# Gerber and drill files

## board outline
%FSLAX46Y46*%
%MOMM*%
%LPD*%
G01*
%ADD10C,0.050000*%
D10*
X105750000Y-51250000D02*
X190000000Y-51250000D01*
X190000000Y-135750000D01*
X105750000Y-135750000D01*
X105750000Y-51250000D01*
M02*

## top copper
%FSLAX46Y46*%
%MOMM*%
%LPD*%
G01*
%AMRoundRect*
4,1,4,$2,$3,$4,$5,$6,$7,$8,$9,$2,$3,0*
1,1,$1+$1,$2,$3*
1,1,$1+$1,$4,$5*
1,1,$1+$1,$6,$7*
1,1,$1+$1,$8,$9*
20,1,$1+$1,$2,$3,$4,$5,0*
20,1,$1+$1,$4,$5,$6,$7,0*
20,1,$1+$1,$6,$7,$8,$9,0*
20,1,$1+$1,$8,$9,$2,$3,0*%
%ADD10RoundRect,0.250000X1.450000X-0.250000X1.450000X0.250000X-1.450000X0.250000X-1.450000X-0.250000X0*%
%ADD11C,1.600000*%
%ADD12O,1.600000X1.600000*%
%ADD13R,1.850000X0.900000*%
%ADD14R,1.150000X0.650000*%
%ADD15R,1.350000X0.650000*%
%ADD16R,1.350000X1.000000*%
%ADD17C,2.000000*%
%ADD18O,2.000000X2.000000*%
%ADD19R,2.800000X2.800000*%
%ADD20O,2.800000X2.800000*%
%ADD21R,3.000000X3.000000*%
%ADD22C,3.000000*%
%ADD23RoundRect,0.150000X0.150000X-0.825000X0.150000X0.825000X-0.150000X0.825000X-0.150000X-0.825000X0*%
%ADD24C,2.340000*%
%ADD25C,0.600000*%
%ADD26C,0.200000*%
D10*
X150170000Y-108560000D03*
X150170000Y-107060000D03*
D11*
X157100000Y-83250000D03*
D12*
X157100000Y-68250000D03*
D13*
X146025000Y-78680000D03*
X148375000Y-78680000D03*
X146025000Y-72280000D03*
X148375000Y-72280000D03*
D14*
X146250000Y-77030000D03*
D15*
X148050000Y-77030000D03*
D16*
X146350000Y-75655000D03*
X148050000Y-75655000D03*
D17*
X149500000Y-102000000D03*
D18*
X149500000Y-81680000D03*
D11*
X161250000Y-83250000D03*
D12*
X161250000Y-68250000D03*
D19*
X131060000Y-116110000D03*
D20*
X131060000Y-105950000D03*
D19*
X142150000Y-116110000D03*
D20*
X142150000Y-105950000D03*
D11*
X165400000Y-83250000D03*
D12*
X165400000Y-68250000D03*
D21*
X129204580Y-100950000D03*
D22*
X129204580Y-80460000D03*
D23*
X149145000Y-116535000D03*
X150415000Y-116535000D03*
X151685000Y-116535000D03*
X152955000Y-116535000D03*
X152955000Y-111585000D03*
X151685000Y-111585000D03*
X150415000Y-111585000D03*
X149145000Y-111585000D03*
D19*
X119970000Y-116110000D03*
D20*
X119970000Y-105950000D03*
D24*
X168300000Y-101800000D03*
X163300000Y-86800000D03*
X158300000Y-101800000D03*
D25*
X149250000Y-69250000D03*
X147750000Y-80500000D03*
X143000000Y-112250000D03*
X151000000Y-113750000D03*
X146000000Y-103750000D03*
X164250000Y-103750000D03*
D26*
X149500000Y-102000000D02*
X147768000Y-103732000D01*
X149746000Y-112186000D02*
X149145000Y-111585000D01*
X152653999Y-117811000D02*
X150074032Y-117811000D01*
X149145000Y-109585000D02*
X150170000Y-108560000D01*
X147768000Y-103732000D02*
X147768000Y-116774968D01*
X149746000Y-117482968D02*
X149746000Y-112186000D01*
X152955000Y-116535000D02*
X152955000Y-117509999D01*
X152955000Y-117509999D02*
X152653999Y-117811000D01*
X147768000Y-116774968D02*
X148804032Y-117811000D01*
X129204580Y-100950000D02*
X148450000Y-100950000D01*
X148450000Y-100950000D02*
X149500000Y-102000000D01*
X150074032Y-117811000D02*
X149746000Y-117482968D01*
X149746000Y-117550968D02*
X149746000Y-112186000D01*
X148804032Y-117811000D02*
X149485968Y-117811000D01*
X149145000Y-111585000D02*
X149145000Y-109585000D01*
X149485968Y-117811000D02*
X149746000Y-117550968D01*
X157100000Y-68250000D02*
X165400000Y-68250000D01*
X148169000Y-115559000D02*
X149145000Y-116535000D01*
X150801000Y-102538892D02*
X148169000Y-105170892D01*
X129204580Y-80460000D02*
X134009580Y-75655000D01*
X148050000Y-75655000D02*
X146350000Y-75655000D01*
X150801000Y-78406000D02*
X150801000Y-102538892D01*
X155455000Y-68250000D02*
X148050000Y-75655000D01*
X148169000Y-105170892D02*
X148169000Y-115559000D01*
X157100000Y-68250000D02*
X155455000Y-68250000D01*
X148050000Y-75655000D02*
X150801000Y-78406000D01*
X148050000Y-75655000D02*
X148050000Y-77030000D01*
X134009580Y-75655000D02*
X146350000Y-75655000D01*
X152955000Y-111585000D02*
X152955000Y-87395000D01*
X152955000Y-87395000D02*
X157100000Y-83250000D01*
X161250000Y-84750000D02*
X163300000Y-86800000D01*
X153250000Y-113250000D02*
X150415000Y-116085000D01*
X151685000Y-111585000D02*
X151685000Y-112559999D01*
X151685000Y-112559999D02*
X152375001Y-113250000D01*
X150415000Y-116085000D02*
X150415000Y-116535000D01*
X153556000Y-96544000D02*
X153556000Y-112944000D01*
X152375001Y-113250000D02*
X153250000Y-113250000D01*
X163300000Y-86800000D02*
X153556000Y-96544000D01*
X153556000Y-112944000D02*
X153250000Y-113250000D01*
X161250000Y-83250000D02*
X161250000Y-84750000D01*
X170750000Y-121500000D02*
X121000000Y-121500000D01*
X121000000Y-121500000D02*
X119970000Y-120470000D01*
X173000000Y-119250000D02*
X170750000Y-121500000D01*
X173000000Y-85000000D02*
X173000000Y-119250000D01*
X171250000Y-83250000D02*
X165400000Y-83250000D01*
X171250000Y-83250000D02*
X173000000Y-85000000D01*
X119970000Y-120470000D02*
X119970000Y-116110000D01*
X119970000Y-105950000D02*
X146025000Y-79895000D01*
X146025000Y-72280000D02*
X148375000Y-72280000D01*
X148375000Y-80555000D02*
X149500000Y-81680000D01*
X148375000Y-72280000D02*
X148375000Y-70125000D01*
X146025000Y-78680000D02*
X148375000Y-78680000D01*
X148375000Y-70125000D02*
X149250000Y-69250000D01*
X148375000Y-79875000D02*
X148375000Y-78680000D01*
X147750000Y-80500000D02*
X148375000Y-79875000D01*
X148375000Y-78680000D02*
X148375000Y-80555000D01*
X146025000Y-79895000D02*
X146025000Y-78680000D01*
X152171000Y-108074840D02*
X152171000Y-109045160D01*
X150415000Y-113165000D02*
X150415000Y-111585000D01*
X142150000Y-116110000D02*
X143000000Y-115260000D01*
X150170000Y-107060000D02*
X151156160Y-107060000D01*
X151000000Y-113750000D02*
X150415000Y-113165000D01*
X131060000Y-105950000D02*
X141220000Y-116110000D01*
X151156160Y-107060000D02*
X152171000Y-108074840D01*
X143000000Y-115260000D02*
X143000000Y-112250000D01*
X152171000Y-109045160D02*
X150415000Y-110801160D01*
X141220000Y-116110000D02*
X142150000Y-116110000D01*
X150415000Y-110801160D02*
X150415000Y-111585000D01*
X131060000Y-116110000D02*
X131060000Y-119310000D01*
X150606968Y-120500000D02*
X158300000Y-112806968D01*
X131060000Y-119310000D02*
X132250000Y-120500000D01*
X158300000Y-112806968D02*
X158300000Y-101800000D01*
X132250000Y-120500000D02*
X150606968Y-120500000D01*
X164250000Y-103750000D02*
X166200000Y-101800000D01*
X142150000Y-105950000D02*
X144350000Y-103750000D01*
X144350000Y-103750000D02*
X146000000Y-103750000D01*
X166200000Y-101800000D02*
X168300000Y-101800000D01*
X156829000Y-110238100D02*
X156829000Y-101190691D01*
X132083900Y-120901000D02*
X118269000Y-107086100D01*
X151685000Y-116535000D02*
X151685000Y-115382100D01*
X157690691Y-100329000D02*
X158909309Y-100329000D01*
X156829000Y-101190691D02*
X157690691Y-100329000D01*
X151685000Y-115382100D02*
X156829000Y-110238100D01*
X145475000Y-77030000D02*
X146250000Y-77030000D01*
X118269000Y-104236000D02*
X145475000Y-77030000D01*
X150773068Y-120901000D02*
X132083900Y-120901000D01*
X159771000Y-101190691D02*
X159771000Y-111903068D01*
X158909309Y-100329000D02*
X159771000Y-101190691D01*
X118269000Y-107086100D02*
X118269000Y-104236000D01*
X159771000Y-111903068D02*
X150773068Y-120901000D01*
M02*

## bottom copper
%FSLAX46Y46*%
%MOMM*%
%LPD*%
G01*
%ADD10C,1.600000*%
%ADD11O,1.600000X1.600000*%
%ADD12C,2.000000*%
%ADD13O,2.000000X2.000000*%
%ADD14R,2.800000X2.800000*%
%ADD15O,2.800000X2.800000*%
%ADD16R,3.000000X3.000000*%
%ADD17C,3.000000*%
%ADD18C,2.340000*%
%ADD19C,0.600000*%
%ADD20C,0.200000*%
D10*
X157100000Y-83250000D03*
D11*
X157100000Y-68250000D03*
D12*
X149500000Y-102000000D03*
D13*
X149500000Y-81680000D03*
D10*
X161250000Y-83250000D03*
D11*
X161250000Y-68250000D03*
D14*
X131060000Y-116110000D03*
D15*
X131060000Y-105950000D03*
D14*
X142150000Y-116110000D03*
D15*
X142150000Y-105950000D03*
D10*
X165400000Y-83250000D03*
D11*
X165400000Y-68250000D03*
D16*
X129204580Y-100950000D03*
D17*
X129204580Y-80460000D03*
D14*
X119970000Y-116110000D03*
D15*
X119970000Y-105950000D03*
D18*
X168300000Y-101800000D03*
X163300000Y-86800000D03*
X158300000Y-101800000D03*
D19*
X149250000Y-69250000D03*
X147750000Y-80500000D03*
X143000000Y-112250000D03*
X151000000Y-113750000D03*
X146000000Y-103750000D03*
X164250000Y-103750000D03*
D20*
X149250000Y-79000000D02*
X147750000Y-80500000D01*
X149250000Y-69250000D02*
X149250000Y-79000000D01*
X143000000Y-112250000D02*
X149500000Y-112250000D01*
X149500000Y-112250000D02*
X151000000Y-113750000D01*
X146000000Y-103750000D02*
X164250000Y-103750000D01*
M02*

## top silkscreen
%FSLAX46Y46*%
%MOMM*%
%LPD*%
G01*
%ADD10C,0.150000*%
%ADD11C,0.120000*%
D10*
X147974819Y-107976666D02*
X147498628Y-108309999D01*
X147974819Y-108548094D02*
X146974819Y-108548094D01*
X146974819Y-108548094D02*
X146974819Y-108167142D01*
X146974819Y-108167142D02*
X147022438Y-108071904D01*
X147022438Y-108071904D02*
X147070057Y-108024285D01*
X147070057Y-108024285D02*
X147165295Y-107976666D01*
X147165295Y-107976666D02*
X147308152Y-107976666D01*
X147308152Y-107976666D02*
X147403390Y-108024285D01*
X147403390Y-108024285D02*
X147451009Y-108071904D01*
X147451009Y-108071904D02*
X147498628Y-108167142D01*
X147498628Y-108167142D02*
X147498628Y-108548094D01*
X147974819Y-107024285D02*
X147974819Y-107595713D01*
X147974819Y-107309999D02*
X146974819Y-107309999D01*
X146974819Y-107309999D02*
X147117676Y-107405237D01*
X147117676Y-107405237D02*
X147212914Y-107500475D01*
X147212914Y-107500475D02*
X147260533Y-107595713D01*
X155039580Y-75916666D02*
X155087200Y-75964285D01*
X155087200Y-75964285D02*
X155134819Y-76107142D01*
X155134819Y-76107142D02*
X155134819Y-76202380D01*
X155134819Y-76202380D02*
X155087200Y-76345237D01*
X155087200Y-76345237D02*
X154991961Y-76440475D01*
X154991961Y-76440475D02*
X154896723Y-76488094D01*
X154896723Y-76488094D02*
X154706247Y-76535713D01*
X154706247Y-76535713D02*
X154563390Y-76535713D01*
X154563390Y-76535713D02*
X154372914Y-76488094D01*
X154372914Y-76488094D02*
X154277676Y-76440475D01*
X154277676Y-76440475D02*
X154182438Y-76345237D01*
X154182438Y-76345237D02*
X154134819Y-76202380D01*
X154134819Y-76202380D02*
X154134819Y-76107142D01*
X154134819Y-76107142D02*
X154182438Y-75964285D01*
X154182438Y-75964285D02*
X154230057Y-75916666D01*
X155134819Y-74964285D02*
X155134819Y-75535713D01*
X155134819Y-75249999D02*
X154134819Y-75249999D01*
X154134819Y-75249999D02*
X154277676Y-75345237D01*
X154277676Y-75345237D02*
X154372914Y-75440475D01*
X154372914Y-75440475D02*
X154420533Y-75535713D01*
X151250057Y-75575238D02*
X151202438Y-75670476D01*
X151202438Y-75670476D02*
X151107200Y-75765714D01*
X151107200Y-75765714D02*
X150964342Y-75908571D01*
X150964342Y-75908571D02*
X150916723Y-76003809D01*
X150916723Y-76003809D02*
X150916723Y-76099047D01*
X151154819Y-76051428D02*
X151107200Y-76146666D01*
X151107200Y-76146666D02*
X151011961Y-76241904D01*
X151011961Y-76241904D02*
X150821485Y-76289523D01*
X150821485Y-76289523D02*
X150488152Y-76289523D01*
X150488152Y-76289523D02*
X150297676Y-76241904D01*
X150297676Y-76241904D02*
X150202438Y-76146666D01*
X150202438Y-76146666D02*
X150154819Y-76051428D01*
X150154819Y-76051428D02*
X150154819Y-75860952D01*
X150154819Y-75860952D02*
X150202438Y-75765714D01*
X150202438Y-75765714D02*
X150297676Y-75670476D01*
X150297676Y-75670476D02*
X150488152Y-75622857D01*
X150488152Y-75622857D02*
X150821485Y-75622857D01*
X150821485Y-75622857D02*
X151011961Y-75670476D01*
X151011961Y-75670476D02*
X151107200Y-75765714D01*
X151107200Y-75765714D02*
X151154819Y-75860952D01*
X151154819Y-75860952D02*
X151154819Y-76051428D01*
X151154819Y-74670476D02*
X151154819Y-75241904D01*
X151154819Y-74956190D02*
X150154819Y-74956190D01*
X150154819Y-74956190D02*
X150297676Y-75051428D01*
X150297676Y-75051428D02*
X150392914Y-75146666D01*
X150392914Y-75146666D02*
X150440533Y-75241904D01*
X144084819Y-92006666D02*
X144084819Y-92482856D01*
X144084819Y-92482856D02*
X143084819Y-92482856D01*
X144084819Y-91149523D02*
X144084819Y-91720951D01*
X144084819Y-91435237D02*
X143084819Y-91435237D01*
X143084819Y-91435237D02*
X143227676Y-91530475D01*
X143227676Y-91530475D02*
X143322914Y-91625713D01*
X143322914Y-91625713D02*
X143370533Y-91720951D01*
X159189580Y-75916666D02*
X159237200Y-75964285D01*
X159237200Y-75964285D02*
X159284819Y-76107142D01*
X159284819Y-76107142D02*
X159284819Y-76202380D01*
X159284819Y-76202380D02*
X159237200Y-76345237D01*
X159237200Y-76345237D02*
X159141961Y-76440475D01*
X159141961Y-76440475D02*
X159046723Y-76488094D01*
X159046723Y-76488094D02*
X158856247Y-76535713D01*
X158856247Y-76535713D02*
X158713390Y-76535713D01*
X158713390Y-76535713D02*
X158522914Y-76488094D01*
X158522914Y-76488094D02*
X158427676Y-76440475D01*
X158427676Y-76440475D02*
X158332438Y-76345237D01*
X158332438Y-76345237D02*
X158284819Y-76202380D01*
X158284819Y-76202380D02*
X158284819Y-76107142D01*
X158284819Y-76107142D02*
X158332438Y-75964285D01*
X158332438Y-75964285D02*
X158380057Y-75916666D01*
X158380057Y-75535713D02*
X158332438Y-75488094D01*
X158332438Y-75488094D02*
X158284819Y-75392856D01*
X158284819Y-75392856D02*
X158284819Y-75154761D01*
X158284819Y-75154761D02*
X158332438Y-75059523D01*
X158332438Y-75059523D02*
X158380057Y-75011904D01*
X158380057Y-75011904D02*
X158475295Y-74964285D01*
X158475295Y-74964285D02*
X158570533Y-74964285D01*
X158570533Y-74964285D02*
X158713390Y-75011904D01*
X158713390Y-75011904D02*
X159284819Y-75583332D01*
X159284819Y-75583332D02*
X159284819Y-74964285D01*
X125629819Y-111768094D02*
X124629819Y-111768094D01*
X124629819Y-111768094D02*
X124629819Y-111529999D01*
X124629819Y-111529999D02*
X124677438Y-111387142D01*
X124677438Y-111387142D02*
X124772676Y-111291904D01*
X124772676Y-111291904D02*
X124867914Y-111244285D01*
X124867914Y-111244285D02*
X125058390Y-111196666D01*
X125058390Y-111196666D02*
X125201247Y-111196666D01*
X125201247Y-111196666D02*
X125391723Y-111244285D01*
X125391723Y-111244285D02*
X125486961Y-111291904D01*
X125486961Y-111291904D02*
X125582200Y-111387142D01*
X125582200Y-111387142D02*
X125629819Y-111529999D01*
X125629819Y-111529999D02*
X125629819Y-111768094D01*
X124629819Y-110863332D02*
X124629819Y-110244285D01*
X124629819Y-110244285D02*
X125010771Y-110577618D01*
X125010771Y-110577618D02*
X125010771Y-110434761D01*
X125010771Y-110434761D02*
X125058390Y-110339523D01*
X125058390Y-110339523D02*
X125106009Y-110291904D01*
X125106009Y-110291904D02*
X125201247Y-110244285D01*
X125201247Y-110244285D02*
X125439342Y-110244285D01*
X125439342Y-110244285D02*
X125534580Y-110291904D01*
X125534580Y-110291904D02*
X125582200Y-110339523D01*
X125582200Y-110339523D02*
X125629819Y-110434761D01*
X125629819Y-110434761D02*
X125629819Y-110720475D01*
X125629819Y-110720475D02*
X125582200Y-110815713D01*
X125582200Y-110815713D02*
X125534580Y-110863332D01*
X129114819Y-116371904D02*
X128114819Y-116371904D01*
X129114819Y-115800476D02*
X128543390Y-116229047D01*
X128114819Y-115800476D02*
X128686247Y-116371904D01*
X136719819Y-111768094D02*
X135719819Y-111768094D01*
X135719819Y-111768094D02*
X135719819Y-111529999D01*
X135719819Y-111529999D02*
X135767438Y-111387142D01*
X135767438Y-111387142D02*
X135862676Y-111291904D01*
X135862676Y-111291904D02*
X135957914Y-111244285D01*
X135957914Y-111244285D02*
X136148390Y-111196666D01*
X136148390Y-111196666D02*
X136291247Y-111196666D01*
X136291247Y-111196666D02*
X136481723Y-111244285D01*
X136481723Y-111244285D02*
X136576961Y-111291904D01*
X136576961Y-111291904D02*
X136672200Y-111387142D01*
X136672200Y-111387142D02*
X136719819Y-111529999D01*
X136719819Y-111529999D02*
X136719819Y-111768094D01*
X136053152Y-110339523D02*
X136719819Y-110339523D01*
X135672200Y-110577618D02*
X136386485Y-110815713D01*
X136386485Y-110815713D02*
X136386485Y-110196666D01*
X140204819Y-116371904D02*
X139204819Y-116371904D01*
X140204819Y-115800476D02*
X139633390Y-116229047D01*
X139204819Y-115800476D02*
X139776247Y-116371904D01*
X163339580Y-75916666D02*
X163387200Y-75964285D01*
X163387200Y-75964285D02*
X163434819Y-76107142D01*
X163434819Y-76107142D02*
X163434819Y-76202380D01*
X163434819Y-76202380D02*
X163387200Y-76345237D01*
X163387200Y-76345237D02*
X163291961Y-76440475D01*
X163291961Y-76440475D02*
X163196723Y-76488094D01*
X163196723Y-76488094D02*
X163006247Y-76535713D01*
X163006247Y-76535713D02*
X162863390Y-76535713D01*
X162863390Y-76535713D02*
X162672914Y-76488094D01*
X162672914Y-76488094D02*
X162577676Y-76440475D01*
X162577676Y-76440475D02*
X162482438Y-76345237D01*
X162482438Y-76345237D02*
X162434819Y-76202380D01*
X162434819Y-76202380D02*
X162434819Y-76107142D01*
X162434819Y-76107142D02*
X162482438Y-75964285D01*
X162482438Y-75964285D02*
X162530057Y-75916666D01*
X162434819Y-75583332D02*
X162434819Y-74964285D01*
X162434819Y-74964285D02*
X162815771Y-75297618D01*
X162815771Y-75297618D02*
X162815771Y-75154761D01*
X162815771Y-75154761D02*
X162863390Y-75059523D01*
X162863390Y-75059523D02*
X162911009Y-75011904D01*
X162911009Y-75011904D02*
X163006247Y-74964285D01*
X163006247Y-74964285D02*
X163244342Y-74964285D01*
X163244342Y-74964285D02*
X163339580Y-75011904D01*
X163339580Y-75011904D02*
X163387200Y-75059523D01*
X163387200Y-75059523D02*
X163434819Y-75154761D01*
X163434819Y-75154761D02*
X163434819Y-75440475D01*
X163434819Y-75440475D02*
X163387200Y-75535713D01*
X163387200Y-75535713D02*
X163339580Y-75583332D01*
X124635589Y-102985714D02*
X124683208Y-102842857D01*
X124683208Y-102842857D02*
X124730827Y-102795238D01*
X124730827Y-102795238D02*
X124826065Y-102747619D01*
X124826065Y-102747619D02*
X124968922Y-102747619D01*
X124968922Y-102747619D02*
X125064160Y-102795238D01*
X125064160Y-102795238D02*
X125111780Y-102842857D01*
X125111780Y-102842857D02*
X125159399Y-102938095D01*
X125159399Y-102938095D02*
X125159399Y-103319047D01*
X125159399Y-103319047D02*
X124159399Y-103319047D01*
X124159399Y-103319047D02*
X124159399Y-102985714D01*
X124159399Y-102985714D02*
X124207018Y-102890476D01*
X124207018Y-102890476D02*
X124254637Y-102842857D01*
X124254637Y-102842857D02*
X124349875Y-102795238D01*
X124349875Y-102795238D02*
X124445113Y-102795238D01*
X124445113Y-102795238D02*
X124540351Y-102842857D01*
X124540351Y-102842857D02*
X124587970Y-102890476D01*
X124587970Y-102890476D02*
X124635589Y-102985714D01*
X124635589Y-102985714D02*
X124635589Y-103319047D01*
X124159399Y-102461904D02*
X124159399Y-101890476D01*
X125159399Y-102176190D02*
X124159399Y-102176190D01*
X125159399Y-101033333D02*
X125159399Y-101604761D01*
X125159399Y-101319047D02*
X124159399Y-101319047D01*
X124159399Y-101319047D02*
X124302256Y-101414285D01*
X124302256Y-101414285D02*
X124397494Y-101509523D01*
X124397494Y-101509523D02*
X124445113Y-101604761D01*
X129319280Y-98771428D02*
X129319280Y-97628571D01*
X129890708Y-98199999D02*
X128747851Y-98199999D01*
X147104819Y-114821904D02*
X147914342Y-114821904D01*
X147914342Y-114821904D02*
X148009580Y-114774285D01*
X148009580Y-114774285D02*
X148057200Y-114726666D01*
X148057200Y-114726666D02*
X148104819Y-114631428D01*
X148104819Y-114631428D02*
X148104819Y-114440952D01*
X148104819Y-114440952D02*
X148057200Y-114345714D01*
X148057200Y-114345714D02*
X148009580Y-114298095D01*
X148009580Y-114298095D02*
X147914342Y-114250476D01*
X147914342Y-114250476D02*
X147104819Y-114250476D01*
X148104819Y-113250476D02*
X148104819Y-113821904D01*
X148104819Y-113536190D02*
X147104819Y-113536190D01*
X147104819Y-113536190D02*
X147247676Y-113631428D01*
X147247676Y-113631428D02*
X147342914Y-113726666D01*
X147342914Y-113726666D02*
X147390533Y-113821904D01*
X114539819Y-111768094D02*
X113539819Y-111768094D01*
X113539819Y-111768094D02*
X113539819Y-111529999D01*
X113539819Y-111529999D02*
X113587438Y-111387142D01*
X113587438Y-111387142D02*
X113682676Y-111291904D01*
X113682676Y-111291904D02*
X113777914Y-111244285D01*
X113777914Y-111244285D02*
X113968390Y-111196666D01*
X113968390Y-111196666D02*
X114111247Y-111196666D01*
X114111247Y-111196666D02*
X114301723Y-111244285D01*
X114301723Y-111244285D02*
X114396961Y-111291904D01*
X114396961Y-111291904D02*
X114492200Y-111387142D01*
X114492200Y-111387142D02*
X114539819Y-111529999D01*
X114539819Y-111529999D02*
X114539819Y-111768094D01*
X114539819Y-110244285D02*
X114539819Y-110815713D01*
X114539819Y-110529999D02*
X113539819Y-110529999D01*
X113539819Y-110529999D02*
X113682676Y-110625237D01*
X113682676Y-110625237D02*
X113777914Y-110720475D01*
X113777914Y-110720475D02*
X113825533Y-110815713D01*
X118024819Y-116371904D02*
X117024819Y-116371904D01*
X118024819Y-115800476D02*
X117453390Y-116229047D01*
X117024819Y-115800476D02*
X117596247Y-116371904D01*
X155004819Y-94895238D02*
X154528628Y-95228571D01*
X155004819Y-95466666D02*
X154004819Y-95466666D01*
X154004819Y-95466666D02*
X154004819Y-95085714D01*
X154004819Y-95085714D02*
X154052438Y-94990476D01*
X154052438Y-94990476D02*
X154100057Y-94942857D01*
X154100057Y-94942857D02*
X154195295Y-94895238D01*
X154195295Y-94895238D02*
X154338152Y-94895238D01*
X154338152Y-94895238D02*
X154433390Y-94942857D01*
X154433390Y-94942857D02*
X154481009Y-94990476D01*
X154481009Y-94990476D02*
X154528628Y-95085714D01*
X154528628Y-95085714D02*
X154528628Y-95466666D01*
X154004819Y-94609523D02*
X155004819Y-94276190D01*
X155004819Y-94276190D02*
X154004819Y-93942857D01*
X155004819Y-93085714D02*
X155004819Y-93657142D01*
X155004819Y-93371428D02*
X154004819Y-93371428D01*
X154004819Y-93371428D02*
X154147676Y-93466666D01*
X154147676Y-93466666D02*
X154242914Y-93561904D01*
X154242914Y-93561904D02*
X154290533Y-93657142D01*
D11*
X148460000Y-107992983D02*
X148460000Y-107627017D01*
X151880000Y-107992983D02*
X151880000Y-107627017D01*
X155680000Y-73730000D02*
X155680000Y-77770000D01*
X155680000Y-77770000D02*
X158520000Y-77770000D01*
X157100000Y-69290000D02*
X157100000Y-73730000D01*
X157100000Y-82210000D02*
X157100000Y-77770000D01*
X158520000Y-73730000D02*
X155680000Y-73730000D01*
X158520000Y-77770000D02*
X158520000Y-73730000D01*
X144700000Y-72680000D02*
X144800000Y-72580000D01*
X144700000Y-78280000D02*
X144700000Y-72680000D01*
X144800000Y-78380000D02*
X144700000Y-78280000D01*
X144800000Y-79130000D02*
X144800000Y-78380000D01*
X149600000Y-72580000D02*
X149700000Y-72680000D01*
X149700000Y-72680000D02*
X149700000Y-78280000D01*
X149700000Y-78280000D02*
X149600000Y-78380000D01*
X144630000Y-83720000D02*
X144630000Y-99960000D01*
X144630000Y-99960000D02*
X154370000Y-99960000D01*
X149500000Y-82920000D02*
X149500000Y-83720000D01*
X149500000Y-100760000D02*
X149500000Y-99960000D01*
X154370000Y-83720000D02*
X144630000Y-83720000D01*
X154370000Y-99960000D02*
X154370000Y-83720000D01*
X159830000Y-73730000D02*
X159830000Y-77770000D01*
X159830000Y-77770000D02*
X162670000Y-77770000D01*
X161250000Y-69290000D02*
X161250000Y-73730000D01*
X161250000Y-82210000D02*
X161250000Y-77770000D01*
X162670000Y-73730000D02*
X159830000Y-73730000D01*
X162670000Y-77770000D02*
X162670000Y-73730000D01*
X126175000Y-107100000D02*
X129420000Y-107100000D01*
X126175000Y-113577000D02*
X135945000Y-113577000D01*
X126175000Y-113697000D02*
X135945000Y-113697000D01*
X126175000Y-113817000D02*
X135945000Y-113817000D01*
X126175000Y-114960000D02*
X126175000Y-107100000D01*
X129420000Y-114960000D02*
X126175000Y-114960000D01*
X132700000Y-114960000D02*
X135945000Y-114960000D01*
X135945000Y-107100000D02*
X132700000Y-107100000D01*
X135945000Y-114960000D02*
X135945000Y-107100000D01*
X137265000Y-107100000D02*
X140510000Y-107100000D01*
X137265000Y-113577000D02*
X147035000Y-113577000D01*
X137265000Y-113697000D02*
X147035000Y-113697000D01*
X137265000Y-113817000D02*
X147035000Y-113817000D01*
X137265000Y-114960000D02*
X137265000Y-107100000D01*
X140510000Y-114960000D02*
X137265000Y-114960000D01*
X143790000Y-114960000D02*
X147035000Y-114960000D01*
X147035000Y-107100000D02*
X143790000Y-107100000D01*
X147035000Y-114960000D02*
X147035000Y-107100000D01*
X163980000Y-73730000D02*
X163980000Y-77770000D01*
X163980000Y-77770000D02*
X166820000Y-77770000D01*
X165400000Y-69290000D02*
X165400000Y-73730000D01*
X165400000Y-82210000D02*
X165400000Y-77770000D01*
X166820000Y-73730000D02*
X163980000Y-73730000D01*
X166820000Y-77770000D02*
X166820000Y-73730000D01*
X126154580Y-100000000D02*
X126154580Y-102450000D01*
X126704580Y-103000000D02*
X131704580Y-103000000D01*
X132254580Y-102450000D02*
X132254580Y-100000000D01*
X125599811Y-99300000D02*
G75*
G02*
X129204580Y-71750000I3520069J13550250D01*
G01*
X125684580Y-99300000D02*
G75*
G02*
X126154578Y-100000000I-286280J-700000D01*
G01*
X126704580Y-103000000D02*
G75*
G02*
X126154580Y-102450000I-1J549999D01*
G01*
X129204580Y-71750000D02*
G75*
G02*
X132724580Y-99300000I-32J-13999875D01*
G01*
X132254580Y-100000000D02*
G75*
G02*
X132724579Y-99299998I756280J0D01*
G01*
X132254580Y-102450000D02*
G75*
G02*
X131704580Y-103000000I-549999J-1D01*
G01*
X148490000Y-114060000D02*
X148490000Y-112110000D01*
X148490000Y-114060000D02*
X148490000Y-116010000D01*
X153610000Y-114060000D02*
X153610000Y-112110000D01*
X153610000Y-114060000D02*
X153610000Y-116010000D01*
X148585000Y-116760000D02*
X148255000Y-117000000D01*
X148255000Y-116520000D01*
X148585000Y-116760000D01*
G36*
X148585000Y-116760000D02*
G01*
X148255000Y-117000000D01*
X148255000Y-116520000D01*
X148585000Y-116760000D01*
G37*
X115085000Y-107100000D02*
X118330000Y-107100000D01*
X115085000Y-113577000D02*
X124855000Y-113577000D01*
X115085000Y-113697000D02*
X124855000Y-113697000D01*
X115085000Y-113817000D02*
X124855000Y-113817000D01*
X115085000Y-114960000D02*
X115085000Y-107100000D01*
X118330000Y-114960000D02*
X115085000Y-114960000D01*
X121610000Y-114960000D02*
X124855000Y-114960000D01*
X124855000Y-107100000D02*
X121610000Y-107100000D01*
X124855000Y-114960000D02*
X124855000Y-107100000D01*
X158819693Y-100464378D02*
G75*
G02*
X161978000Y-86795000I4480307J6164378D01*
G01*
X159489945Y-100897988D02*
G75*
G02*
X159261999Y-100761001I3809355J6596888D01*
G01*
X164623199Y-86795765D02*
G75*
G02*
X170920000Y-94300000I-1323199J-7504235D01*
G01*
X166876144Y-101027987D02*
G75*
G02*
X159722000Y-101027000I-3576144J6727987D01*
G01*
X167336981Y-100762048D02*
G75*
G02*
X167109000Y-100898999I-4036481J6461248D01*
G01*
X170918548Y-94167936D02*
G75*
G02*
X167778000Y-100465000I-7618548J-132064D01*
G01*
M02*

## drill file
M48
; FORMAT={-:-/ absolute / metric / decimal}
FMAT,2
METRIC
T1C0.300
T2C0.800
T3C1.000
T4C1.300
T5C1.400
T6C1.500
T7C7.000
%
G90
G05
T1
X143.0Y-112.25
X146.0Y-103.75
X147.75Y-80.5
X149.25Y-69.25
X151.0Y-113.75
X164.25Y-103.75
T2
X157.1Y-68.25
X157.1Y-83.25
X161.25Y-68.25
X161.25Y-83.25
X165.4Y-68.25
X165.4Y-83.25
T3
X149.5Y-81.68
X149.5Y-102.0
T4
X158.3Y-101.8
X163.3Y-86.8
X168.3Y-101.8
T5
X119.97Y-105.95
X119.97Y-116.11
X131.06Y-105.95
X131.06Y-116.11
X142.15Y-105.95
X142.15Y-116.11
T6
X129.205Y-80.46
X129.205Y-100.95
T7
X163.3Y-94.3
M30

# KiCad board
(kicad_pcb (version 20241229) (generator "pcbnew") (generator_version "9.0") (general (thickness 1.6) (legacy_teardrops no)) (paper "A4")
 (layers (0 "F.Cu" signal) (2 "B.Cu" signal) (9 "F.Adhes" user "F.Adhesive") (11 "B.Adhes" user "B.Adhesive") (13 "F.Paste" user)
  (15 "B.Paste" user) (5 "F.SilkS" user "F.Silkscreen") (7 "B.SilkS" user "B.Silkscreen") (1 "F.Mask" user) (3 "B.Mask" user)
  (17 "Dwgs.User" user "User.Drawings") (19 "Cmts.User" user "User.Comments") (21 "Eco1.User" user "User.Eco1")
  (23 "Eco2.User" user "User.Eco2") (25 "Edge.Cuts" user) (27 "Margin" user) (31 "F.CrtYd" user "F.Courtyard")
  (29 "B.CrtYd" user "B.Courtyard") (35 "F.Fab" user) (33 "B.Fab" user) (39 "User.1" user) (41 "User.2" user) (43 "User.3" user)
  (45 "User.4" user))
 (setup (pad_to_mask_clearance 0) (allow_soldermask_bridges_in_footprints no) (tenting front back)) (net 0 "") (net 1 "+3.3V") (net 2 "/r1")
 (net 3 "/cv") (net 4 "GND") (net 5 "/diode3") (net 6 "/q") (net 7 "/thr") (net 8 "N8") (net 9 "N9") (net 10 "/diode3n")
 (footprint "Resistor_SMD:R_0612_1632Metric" (layer "F.Cu") (at 150.17 107.81 90)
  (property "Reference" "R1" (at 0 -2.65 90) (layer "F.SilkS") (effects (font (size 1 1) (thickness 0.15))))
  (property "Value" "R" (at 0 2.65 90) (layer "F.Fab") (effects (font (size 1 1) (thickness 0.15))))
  (fp_line (start -0.182983 -1.71) (end 0.182983 -1.71) (stroke (width 0.12) (type solid)) (layer "F.SilkS"))
  (fp_line (start -0.182983 1.71) (end 0.182983 1.71) (stroke (width 0.12) (type solid)) (layer "F.SilkS"))
  (pad "1" smd roundrect (at -0.75 0 90) (size 1 3.4) (layers "F.Cu" "F.Mask" "F.Paste") (roundrect_rratio 0.25) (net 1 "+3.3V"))
  (pad "2" smd roundrect (at 0.75 0 90) (size 1 3.4) (layers "F.Cu" "F.Mask" "F.Paste") (roundrect_rratio 0.25) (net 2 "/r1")))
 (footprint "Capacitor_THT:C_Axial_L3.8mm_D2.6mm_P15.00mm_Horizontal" (layer "F.Cu") (at 157.1 83.25 90)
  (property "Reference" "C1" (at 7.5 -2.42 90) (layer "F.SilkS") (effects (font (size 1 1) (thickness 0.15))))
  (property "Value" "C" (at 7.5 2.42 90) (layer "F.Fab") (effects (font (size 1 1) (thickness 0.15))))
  (fp_line (start 9.52 -1.42) (end 5.48 -1.42) (stroke (width 0.12) (type solid)) (layer "F.SilkS"))
  (fp_line (start 5.48 -1.42) (end 5.48 1.42) (stroke (width 0.12) (type solid)) (layer "F.SilkS"))
  (fp_line (start 13.96 0) (end 9.52 0) (stroke (width 0.12) (type solid)) (layer "F.SilkS"))
  (fp_line (start 1.04 0) (end 5.48 0) (stroke (width 0.12) (type solid)) (layer "F.SilkS"))
  (fp_line (start 9.52 1.42) (end 9.52 -1.42) (stroke (width 0.12) (type solid)) (layer "F.SilkS"))
  (fp_line (start 5.48 1.42) (end 9.52 1.42) (stroke (width 0.12) (type solid)) (layer "F.SilkS"))
  (pad "1" thru_hole circle (at 0 0 90) (size 1.6 1.6) (drill 0.8) (layers "*.Cu" "*.Mask") (remove_unused_layers no) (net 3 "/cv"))
  (pad "2" thru_hole oval (at 15 0 90) (size 1.6 1.6) (drill 0.8) (layers "*.Cu" "*.Mask") (remove_unused_layers no) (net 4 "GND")))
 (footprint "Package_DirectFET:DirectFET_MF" (layer "F.Cu") (at 147.2 75.48 90)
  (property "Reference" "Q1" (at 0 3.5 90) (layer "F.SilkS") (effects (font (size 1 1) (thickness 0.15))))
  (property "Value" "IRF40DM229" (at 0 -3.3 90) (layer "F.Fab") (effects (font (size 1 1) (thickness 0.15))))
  (fp_line (start 2.8 -2.5) (end 2.9 -2.4) (stroke (width 0.12) (type solid)) (layer "F.SilkS"))
  (fp_line (start -2.8 -2.5) (end 2.8 -2.5) (stroke (width 0.12) (type solid)) (layer "F.SilkS"))
  (fp_line (start -2.9 -2.4) (end -2.8 -2.5) (stroke (width 0.12) (type solid)) (layer "F.SilkS"))
  (fp_line (start -3.65 -2.4) (end -2.9 -2.4) (stroke (width 0.12) (type solid)) (layer "F.SilkS"))
  (fp_line (start 2.9 2.4) (end 2.8 2.5) (stroke (width 0.12) (type solid)) (layer "F.SilkS"))
  (fp_line (start 2.8 2.5) (end -2.8 2.5) (stroke (width 0.12) (type solid)) (layer "F.SilkS"))
  (fp_line (start -2.8 2.5) (end -2.9 2.4) (stroke (width 0.12) (type solid)) (layer "F.SilkS"))
  (pad "1" smd rect (at -3.2 -1.175 90) (size 0.9 1.85) (layers "F.Cu" "F.Mask" "F.Paste") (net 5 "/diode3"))
  (pad "1" smd rect (at -3.2 1.175 90) (size 0.9 1.85) (layers "F.Cu" "F.Mask" "F.Paste") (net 5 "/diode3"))
  (pad "1" smd rect (at 3.2 -1.175 90) (size 0.9 1.85) (layers "F.Cu" "F.Mask" "F.Paste") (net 5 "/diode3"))
  (pad "1" smd rect (at 3.2 1.175 90) (size 0.9 1.85) (layers "F.Cu" "F.Mask" "F.Paste") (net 5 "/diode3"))
  (pad "2" smd rect (at -1.55 -0.95 90) (size 0.65 1.15) (layers "F.Cu" "F.Mask" "F.Paste") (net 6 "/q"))
  (pad "3" smd rect (at -1.55 0.85 90) (size 0.65 1.35) (layers "F.Cu" "F.Mask" "F.Paste") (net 4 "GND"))
  (pad "3" smd rect (at -0.175 -0.85 90) (size 1 1.35) (layers "F.Cu" "F.Mask" "F.Paste") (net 4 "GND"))
  (pad "3" smd rect (at -0.175 0.85 90) (size 1 1.35) (layers "F.Cu" "F.Mask" "F.Paste") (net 4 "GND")))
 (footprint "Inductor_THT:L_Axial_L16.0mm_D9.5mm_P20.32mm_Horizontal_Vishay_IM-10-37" (layer "F.Cu") (at 149.5 102 90)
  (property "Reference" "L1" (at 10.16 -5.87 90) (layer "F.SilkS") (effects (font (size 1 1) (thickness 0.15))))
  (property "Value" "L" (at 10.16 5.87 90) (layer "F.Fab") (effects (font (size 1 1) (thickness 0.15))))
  (fp_line (start 18.28 -4.87) (end 2.04 -4.87) (stroke (width 0.12) (type solid)) (layer "F.SilkS"))
  (fp_line (start 2.04 -4.87) (end 2.04 4.87) (stroke (width 0.12) (type solid)) (layer "F.SilkS"))
  (fp_line (start 19.08 0) (end 18.28 0) (stroke (width 0.12) (type solid)) (layer "F.SilkS"))
  (fp_line (start 1.24 0) (end 2.04 0) (stroke (width 0.12) (type solid)) (layer "F.SilkS"))
  (fp_line (start 18.28 4.87) (end 18.28 -4.87) (stroke (width 0.12) (type solid)) (layer "F.SilkS"))
  (fp_line (start 2.04 4.87) (end 18.28 4.87) (stroke (width 0.12) (type solid)) (layer "F.SilkS"))
  (pad "1" thru_hole circle (at 0 0 90) (size 2 2) (drill 1) (layers "*.Cu" "*.Mask") (remove_unused_layers no) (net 1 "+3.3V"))
  (pad "2" thru_hole oval (at 20.32 0 90) (size 2 2) (drill 1) (layers "*.Cu" "*.Mask") (remove_unused_layers no) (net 5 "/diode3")))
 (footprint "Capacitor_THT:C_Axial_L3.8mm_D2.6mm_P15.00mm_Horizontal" (layer "F.Cu") (at 161.25 83.25 90)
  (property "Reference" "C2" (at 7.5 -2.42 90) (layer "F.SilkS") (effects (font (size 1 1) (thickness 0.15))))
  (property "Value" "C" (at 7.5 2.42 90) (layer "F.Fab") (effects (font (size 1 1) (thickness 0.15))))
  (fp_line (start 9.52 -1.42) (end 5.48 -1.42) (stroke (width 0.12) (type solid)) (layer "F.SilkS"))
  (fp_line (start 5.48 -1.42) (end 5.48 1.42) (stroke (width 0.12) (type solid)) (layer "F.SilkS"))
  (fp_line (start 13.96 0) (end 9.52 0) (stroke (width 0.12) (type solid)) (layer "F.SilkS"))
  (fp_line (start 1.04 0) (end 5.48 0) (stroke (width 0.12) (type solid)) (layer "F.SilkS"))
  (fp_line (start 9.52 1.42) (end 9.52 -1.42) (stroke (width 0.12) (type solid)) (layer "F.SilkS"))
  (fp_line (start 5.48 1.42) (end 9.52 1.42) (stroke (width 0.12) (type solid)) (layer "F.SilkS"))
  (pad "1" thru_hole circle (at 0 0 90) (size 1.6 1.6) (drill 0.8) (layers "*.Cu" "*.Mask") (remove_unused_layers no) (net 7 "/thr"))
  (pad "2" thru_hole oval (at 15 0 90) (size 1.6 1.6) (drill 0.8) (layers "*.Cu" "*.Mask") (remove_unused_layers no) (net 4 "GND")))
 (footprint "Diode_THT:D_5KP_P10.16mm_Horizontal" (layer "F.Cu") (at 131.06 116.11 90)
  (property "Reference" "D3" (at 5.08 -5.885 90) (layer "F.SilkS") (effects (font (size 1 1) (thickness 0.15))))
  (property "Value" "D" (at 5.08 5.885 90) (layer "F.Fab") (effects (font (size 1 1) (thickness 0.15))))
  (fp_line (start 9.01 -4.885) (end 9.01 -1.64) (stroke (width 0.12) (type solid)) (layer "F.SilkS"))
  (fp_line (start 2.533 -4.885) (end 2.533 4.885) (stroke (width 0.12) (type solid)) (layer "F.SilkS"))
  (fp_line (start 2.413 -4.885) (end 2.413 4.885) (stroke (width 0.12) (type solid)) (layer "F.SilkS"))
  (fp_line (start 2.293 -4.885) (end 2.293 4.885) (stroke (width 0.12) (type solid)) (layer "F.SilkS"))
  (fp_line (start 1.15 -4.885) (end 9.01 -4.885) (stroke (width 0.12) (type solid)) (layer "F.SilkS"))
  (fp_line (start 1.15 -1.64) (end 1.15 -4.885) (stroke (width 0.12) (type solid)) (layer "F.SilkS"))
  (fp_line (start 1.15 1.64) (end 1.15 4.885) (stroke (width 0.12) (type solid)) (layer "F.SilkS"))
  (fp_line (start 9.01 4.885) (end 9.01 1.64) (stroke (width 0.12) (type solid)) (layer "F.SilkS"))
  (fp_line (start 1.15 4.885) (end 9.01 4.885) (stroke (width 0.12) (type solid)) (layer "F.SilkS"))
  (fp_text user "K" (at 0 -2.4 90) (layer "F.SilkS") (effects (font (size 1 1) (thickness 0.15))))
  (pad "1" thru_hole rect (at 0 0 90) (size 2.8 2.8) (drill 1.4) (layers "*.Cu" "*.Mask") (remove_unused_layers no) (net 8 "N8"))
  (pad "2" thru_hole oval (at 10.16 0 90) (size 2.8 2.8) (drill 1.4) (layers "*.Cu" "*.Mask") (remove_unused_layers no) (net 2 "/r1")))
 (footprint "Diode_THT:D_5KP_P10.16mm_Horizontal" (layer "F.Cu") (at 142.15 116.11 90)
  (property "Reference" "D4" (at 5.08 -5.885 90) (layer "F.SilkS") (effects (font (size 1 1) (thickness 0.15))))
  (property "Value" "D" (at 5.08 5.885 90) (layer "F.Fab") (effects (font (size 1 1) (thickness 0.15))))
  (fp_line (start 9.01 -4.885) (end 9.01 -1.64) (stroke (width 0.12) (type solid)) (layer "F.SilkS"))
  (fp_line (start 2.533 -4.885) (end 2.533 4.885) (stroke (width 0.12) (type solid)) (layer "F.SilkS"))
  (fp_line (start 2.413 -4.885) (end 2.413 4.885) (stroke (width 0.12) (type solid)) (layer "F.SilkS"))
  (fp_line (start 2.293 -4.885) (end 2.293 4.885) (stroke (width 0.12) (type solid)) (layer "F.SilkS"))
  (fp_line (start 1.15 -4.885) (end 9.01 -4.885) (stroke (width 0.12) (type solid)) (layer "F.SilkS"))
  (fp_line (start 1.15 -1.64) (end 1.15 -4.885) (stroke (width 0.12) (type solid)) (layer "F.SilkS"))
  (fp_line (start 1.15 1.64) (end 1.15 4.885) (stroke (width 0.12) (type solid)) (layer "F.SilkS"))
  (fp_line (start 9.01 4.885) (end 9.01 1.64) (stroke (width 0.12) (type solid)) (layer "F.SilkS"))
  (fp_line (start 1.15 4.885) (end 9.01 4.885) (stroke (width 0.12) (type solid)) (layer "F.SilkS"))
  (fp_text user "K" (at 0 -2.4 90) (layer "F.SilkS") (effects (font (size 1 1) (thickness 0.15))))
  (pad "1" thru_hole rect (at 0 0 90) (size 2.8 2.8) (drill 1.4) (layers "*.Cu" "*.Mask") (remove_unused_layers no) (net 2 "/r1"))
  (pad "2" thru_hole oval (at 10.16 0 90) (size 2.8 2.8) (drill 1.4) (layers "*.Cu" "*.Mask") (remove_unused_layers no) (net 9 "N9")))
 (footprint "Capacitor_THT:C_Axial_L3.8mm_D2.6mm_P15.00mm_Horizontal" (layer "F.Cu") (at 165.4 83.25 90)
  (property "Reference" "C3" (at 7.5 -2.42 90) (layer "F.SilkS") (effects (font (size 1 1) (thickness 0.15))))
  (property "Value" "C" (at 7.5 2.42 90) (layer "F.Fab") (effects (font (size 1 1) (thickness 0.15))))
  (fp_line (start 9.52 -1.42) (end 5.48 -1.42) (stroke (width 0.12) (type solid)) (layer "F.SilkS"))
  (fp_line (start 5.48 -1.42) (end 5.48 1.42) (stroke (width 0.12) (type solid)) (layer "F.SilkS"))
  (fp_line (start 13.96 0) (end 9.52 0) (stroke (width 0.12) (type solid)) (layer "F.SilkS"))
  (fp_line (start 1.04 0) (end 5.48 0) (stroke (width 0.12) (type solid)) (layer "F.SilkS"))
  (fp_line (start 9.52 1.42) (end 9.52 -1.42) (stroke (width 0.12) (type solid)) (layer "F.SilkS"))
  (fp_line (start 5.48 1.42) (end 9.52 1.42) (stroke (width 0.12) (type solid)) (layer "F.SilkS"))
  (pad "1" thru_hole circle (at 0 0 90) (size 1.6 1.6) (drill 0.8) (layers "*.Cu" "*.Mask") (remove_unused_layers no) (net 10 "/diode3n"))
  (pad "2" thru_hole oval (at 15 0 90) (size 1.6 1.6) (drill 0.8) (layers "*.Cu" "*.Mask") (remove_unused_layers no) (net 4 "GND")))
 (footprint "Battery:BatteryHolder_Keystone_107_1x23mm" (layer "F.Cu") (at 129.20458 100.95 90)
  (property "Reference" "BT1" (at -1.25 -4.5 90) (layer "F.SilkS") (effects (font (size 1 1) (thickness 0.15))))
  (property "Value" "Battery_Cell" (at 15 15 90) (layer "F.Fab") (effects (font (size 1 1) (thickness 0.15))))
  (fp_line (start 0.95 -3.05) (end -1.5 -3.05) (stroke (width 0.12) (type solid)) (layer "F.SilkS"))
  (fp_line (start -2.05 -2.5) (end -2.05 2.5) (stroke (width 0.12) (type solid)) (layer "F.SilkS"))
  (fp_line (start -1.5 3.05) (end 0.95 3.05) (stroke (width 0.12) (type solid)) (layer "F.SilkS"))
  (fp_arc (start 1.65 -3.604769) (mid 17.016593 -13.966381) (end 29.2 0) (stroke (width 0.12) (type solid)) (layer "F.SilkS"))
  (fp_arc (start 1.65 -3.52) (mid 1.371575 -3.1784) (end 0.95 -3.05) (stroke (width 0.12) (type solid)) (layer "F.SilkS"))
  (fp_arc (start -2.05 -2.5) (mid -1.888909 -2.888909) (end -1.5 -3.05) (stroke (width 0.12) (type solid)) (layer "F.SilkS"))
  (fp_arc (start 29.2 0) (mid 16.974433 13.886952) (end 1.65 3.52) (stroke (width 0.12) (type solid)) (layer "F.SilkS"))
  (fp_arc (start 0.95 3.05) (mid 1.371574 3.1784) (end 1.65 3.52) (stroke (width 0.12) (type solid)) (layer "F.SilkS"))
  (fp_arc (start -1.5 3.05) (mid -1.888909 2.888909) (end -2.05 2.5) (stroke (width 0.12) (type solid)) (layer "F.SilkS"))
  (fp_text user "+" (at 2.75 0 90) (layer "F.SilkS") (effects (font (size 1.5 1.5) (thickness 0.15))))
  (pad "1" thru_hole rect (at 0 0 90) (size 3 3) (drill 1.5) (layers "*.Cu" "*.Mask") (remove_unused_layers no) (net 1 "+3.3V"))
  (pad "2" thru_hole circle (at 20.49 0 90) (size 3 3) (drill 1.5) (layers "*.Cu" "*.Mask") (remove_unused_layers no) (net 4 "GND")))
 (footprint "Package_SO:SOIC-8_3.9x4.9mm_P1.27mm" (layer "F.Cu") (at 151.05 114.06 90)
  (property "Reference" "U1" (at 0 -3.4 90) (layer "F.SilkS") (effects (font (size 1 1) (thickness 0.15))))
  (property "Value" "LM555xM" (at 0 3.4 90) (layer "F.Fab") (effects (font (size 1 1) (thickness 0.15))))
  (fp_line (start 0 -2.56) (end 1.95 -2.56) (stroke (width 0.12) (type solid)) (layer "F.SilkS"))
  (fp_line (start 0 -2.56) (end -1.95 -2.56) (stroke (width 0.12) (type solid)) (layer "F.SilkS"))
  (fp_line (start 0 2.56) (end 1.95 2.56) (stroke (width 0.12) (type solid)) (layer "F.SilkS"))
  (fp_line (start 0 2.56) (end -1.95 2.56) (stroke (width 0.12) (type solid)) (layer "F.SilkS"))
  (fp_poly
   (pts (xy -2.7 -2.465) (xy -2.94 -2.795) (xy -2.46 -2.795) (xy -2.7 -2.465)) (stroke (width 0.12) (type solid)) (fill yes)
   (layer "F.SilkS"))
  (pad "1" smd roundrect (at -2.475 -1.905 90) (size 1.95 0.6) (layers "F.Cu" "F.Mask" "F.Paste") (roundrect_rratio 0.25) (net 4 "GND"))
  (pad "2" smd roundrect (at -2.475 -0.635 90) (size 1.95 0.6) (layers "F.Cu" "F.Mask" "F.Paste") (roundrect_rratio 0.25) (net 7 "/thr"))
  (pad "3" smd roundrect (at -2.475 0.635 90) (size 1.95 0.6) (layers "F.Cu" "F.Mask" "F.Paste") (roundrect_rratio 0.25) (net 6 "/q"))
  (pad "4" smd roundrect (at -2.475 1.905 90) (size 1.95 0.6) (layers "F.Cu" "F.Mask" "F.Paste") (roundrect_rratio 0.25) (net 1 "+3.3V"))
  (pad "5" smd roundrect (at 2.475 1.905 90) (size 1.95 0.6) (layers "F.Cu" "F.Mask" "F.Paste") (roundrect_rratio 0.25) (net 3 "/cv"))
  (pad "6" smd roundrect (at 2.475 0.635 90) (size 1.95 0.6) (layers "F.Cu" "F.Mask" "F.Paste") (roundrect_rratio 0.25) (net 7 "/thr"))
  (pad "7" smd roundrect (at 2.475 -0.635 90) (size 1.95 0.6) (layers "F.Cu" "F.Mask" "F.Paste") (roundrect_rratio 0.25) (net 2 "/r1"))
  (pad "8" smd roundrect (at 2.475 -1.905 90) (size 1.95 0.6) (layers "F.Cu" "F.Mask" "F.Paste") (roundrect_rratio 0.25) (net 1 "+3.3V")))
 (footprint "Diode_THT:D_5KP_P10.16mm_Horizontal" (layer "F.Cu") (at 119.97 116.11 90)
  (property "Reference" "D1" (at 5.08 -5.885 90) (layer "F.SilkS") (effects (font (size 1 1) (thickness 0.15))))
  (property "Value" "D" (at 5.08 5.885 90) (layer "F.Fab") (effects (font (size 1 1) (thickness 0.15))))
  (fp_line (start 9.01 -4.885) (end 9.01 -1.64) (stroke (width 0.12) (type solid)) (layer "F.SilkS"))
  (fp_line (start 2.533 -4.885) (end 2.533 4.885) (stroke (width 0.12) (type solid)) (layer "F.SilkS"))
  (fp_line (start 2.413 -4.885) (end 2.413 4.885) (stroke (width 0.12) (type solid)) (layer "F.SilkS"))
  (fp_line (start 2.293 -4.885) (end 2.293 4.885) (stroke (width 0.12) (type solid)) (layer "F.SilkS"))
  (fp_line (start 1.15 -4.885) (end 9.01 -4.885) (stroke (width 0.12) (type solid)) (layer "F.SilkS"))
  (fp_line (start 1.15 -1.64) (end 1.15 -4.885) (stroke (width 0.12) (type solid)) (layer "F.SilkS"))
  (fp_line (start 1.15 1.64) (end 1.15 4.885) (stroke (width 0.12) (type solid)) (layer "F.SilkS"))
  (fp_line (start 9.01 4.885) (end 9.01 1.64) (stroke (width 0.12) (type solid)) (layer "F.SilkS"))
  (fp_line (start 1.15 4.885) (end 9.01 4.885) (stroke (width 0.12) (type solid)) (layer "F.SilkS"))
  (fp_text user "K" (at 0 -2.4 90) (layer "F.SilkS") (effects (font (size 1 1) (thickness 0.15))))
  (pad "1" thru_hole rect (at 0 0 90) (size 2.8 2.8) (drill 1.4) (layers "*.Cu" "*.Mask") (remove_unused_layers no) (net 10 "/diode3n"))
  (pad "2" thru_hole oval (at 10.16 0 90) (size 2.8 2.8) (drill 1.4) (layers "*.Cu" "*.Mask") (remove_unused_layers no) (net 5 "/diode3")))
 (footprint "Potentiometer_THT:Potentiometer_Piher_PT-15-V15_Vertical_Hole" (layer "F.Cu") (at 168.3 101.8 90)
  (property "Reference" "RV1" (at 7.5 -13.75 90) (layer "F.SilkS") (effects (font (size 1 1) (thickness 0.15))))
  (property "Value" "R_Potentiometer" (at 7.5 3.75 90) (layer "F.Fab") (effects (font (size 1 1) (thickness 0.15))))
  (fp_arc (start 1.335622 -9.480307) (mid 9.21553 -12.424935) (end 15.005 -6.322) (stroke (width 0.12) (type solid)) (layer "F.SilkS"))
  (fp_arc (start 0.902012 -8.810055) (mid 0.969511 -8.924625) (end 1.039 -9.038) (stroke (width 0.12) (type solid)) (layer "F.SilkS"))
  (fp_arc (start 15.004235 -3.676801) (mid 12.398042 0.837259) (end 7.5 2.62) (stroke (width 0.12) (type solid)) (layer "F.SilkS"))
  (fp_arc (start 0.772013 -1.423856) (mid -0.119358 -5.001051) (end 0.773 -8.578) (stroke (width 0.12) (type solid)) (layer "F.SilkS"))
  (fp_arc (start 1.037952 -0.963019) (mid 0.968481 -1.076412) (end 0.901 -1.191) (stroke (width 0.12) (type solid)) (layer "F.SilkS"))
  (fp_arc (start 7.632064 2.618548) (mid 4.099288 1.818715) (end 1.335 -0.522) (stroke (width 0.12) (type solid)) (layer "F.SilkS"))
  (pad "" np_thru_hole circle (at 7.5 -5 90) (size 7 7) (drill 7) (layers "*.Cu" "*.Mask"))
  (pad "1" thru_hole circle (at 0 0 90) (size 2.34 2.34) (drill 1.3) (layers "*.Cu" "*.Mask") (remove_unused_layers no) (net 9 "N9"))
  (pad "2" thru_hole circle (at 15 -5 90) (size 2.34 2.34) (drill 1.3) (layers "*.Cu" "*.Mask") (remove_unused_layers no) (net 7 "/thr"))
  (pad "3" thru_hole circle (at 0 -10 90) (size 2.34 2.34) (drill 1.3) (layers "*.Cu" "*.Mask") (remove_unused_layers no) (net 8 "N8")))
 (gr_rect (start 105.75 51.25) (end 190 135.75) (stroke (width 0.05) (type default)) (fill no) (layer "Edge.Cuts"))
 (segment (start 149.5 102) (end 147.768 103.732) (width 0.2) (layer "F.Cu") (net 1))
 (segment (start 149.746 112.186) (end 149.145 111.585) (width 0.2) (layer "F.Cu") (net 1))
 (segment (start 152.653999 117.811) (end 150.074032 117.811) (width 0.2) (layer "F.Cu") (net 1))
 (segment (start 149.145 109.585) (end 150.17 108.56) (width 0.2) (layer "F.Cu") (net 1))
 (segment (start 147.768 103.732) (end 147.768 116.774968) (width 0.2) (layer "F.Cu") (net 1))
 (segment (start 149.746 117.482968) (end 149.746 112.186) (width 0.2) (layer "F.Cu") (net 1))
 (segment (start 152.955 116.535) (end 152.955 117.509999) (width 0.2) (layer "F.Cu") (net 1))
 (segment (start 152.955 117.509999) (end 152.653999 117.811) (width 0.2) (layer "F.Cu") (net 1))
 (segment (start 147.768 116.774968) (end 148.804032 117.811) (width 0.2) (layer "F.Cu") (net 1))
 (segment (start 129.20458 100.95) (end 148.45 100.95) (width 0.2) (layer "F.Cu") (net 1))
 (segment (start 148.45 100.95) (end 149.5 102) (width 0.2) (layer "F.Cu") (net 1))
 (segment (start 150.074032 117.811) (end 149.746 117.482968) (width 0.2) (layer "F.Cu") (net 1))
 (segment (start 149.746 117.550968) (end 149.746 112.186) (width 0.2) (layer "F.Cu") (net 1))
 (segment (start 148.804032 117.811) (end 149.485968 117.811) (width 0.2) (layer "F.Cu") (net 1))
 (segment (start 149.145 111.585) (end 149.145 109.585) (width 0.2) (layer "F.Cu") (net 1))
 (segment (start 149.485968 117.811) (end 149.746 117.550968) (width 0.2) (layer "F.Cu") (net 1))
 (segment (start 157.1 68.25) (end 165.4 68.25) (width 0.2) (layer "F.Cu") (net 4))
 (segment (start 148.169 115.559) (end 149.145 116.535) (width 0.2) (layer "F.Cu") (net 4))
 (segment (start 150.801 102.538892) (end 148.169 105.170892) (width 0.2) (layer "F.Cu") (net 4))
 (segment (start 129.20458 80.46) (end 134.00958 75.655) (width 0.2) (layer "F.Cu") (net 4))
 (segment (start 148.05 75.655) (end 146.35 75.655) (width 0.2) (layer "F.Cu") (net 4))
 (segment (start 150.801 78.406) (end 150.801 102.538892) (width 0.2) (layer "F.Cu") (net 4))
 (segment (start 155.455 68.25) (end 148.05 75.655) (width 0.2) (layer "F.Cu") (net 4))
 (segment (start 148.169 105.170892) (end 148.169 115.559) (width 0.2) (layer "F.Cu") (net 4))
 (segment (start 157.1 68.25) (end 155.455 68.25) (width 0.2) (layer "F.Cu") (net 4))
 (segment (start 148.05 75.655) (end 150.801 78.406) (width 0.2) (layer "F.Cu") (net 4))
 (segment (start 148.05 75.655) (end 148.05 77.03) (width 0.2) (layer "F.Cu") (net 4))
 (segment (start 134.00958 75.655) (end 146.35 75.655) (width 0.2) (layer "F.Cu") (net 4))
 (segment (start 152.955 111.585) (end 152.955 87.395) (width 0.2) (layer "F.Cu") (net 3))
 (segment (start 152.955 87.395) (end 157.1 83.25) (width 0.2) (layer "F.Cu") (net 3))
 (segment (start 161.25 84.75) (end 163.3 86.8) (width 0.2) (layer "F.Cu") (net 7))
 (segment (start 153.25 113.25) (end 150.415 116.085) (width 0.2) (layer "F.Cu") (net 7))
 (segment (start 151.685 111.585) (end 151.685 112.559999) (width 0.2) (layer "F.Cu") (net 7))
 (segment (start 151.685 112.559999) (end 152.375001 113.25) (width 0.2) (layer "F.Cu") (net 7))
 (segment (start 150.415 116.085) (end 150.415 116.535) (width 0.2) (layer "F.Cu") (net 7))
 (segment (start 153.556 96.544) (end 153.556 112.944) (width 0.2) (layer "F.Cu") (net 7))
 (segment (start 152.375001 113.25) (end 153.25 113.25) (width 0.2) (layer "F.Cu") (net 7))
 (segment (start 163.3 86.8) (end 153.556 96.544) (width 0.2) (layer "F.Cu") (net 7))
 (segment (start 153.556 112.944) (end 153.25 113.25) (width 0.2) (layer "F.Cu") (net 7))
 (segment (start 161.25 83.25) (end 161.25 84.75) (width 0.2) (layer "F.Cu") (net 7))
 (segment (start 170.75 121.5) (end 121 121.5) (width 0.2) (layer "F.Cu") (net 10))
 (segment (start 121 121.5) (end 119.97 120.47) (width 0.2) (layer "F.Cu") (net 10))
 (segment (start 173 119.25) (end 170.75 121.5) (width 0.2) (layer "F.Cu") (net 10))
 (segment (start 173 85) (end 173 119.25) (width 0.2) (layer "F.Cu") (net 10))
 (segment (start 171.25 83.25) (end 165.4 83.25) (width 0.2) (layer "F.Cu") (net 10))
 (segment (start 171.25 83.25) (end 173 85) (width 0.2) (layer "F.Cu") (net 10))
 (segment (start 119.97 120.47) (end 119.97 116.11) (width 0.2) (layer "F.Cu") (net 10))
 (segment (start 119.97 105.95) (end 146.025 79.895) (width 0.2) (layer "F.Cu") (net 5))
 (segment (start 146.025 72.28) (end 148.375 72.28) (width 0.2) (layer "F.Cu") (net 5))
 (segment (start 148.375 80.555) (end 149.5 81.68) (width 0.2) (layer "F.Cu") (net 5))
 (segment (start 148.375 72.28) (end 148.375 70.125) (width 0.2) (layer "F.Cu") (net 5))
 (segment (start 146.025 78.68) (end 148.375 78.68) (width 0.2) (layer "F.Cu") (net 5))
 (segment (start 148.375 70.125) (end 149.25 69.25) (width 0.2) (layer "F.Cu") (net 5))
 (segment (start 148.375 79.875) (end 148.375 78.68) (width 0.2) (layer "F.Cu") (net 5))
 (segment (start 147.75 80.5) (end 148.375 79.875) (width 0.2) (layer "F.Cu") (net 5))
 (segment (start 148.375 78.68) (end 148.375 80.555) (width 0.2) (layer "F.Cu") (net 5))
 (segment (start 146.025 79.895) (end 146.025 78.68) (width 0.2) (layer "F.Cu") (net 5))
 (via (at 149.25 69.25) (size 0.6) (drill 0.3) (layers "F.Cu" "B.Cu") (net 5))
 (via (at 147.75 80.5) (size 0.6) (drill 0.3) (layers "F.Cu" "B.Cu") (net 5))
 (segment (start 149.25 79) (end 147.75 80.5) (width 0.2) (layer "B.Cu") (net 5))
 (segment (start 149.25 69.25) (end 149.25 79) (width 0.2) (layer "B.Cu") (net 5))
 (segment (start 152.171 108.07484) (end 152.171 109.04516) (width 0.2) (layer "F.Cu") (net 2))
 (segment (start 150.415 113.165) (end 150.415 111.585) (width 0.2) (layer "F.Cu") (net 2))
 (segment (start 142.15 116.11) (end 143 115.26) (width 0.2) (layer "F.Cu") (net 2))
 (segment (start 150.17 107.06) (end 151.15616 107.06) (width 0.2) (layer "F.Cu") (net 2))
 (segment (start 151 113.75) (end 150.415 113.165) (width 0.2) (layer "F.Cu") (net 2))
 (segment (start 131.06 105.95) (end 141.22 116.11) (width 0.2) (layer "F.Cu") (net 2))
 (segment (start 151.15616 107.06) (end 152.171 108.07484) (width 0.2) (layer "F.Cu") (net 2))
 (segment (start 143 115.26) (end 143 112.25) (width 0.2) (layer "F.Cu") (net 2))
 (segment (start 152.171 109.04516) (end 150.415 110.80116) (width 0.2) (layer "F.Cu") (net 2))
 (segment (start 141.22 116.11) (end 142.15 116.11) (width 0.2) (layer "F.Cu") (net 2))
 (segment (start 150.415 110.80116) (end 150.415 111.585) (width 0.2) (layer "F.Cu") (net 2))
 (via (at 143 112.25) (size 0.6) (drill 0.3) (layers "F.Cu" "B.Cu") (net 2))
 (via (at 151 113.75) (size 0.6) (drill 0.3) (layers "F.Cu" "B.Cu") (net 2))
 (segment (start 143 112.25) (end 149.5 112.25) (width 0.2) (layer "B.Cu") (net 2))
 (segment (start 149.5 112.25) (end 151 113.75) (width 0.2) (layer "B.Cu") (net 2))
 (segment (start 131.06 116.11) (end 131.06 119.31) (width 0.2) (layer "F.Cu") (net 8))
 (segment (start 150.606968 120.5) (end 158.3 112.806968) (width 0.2) (layer "F.Cu") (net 8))
 (segment (start 131.06 119.31) (end 132.25 120.5) (width 0.2) (layer "F.Cu") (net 8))
 (segment (start 158.3 112.806968) (end 158.3 101.8) (width 0.2) (layer "F.Cu") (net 8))
 (segment (start 132.25 120.5) (end 150.606968 120.5) (width 0.2) (layer "F.Cu") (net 8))
 (segment (start 164.25 103.75) (end 166.2 101.8) (width 0.2) (layer "F.Cu") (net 9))
 (segment (start 142.15 105.95) (end 144.35 103.75) (width 0.2) (layer "F.Cu") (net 9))
 (segment (start 144.35 103.75) (end 146 103.75) (width 0.2) (layer "F.Cu") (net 9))
 (segment (start 166.2 101.8) (end 168.3 101.8) (width 0.2) (layer "F.Cu") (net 9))
 (via (at 146 103.75) (size 0.6) (drill 0.3) (layers "F.Cu" "B.Cu") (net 9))
 (via (at 164.25 103.75) (size 0.6) (drill 0.3) (layers "F.Cu" "B.Cu") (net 9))
 (segment (start 146 103.75) (end 164.25 103.75) (width 0.2) (layer "B.Cu") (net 9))
 (segment (start 156.829 110.2381) (end 156.829 101.190691) (width 0.2) (layer "F.Cu") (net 6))
 (segment (start 132.0839 120.901) (end 118.269 107.0861) (width 0.2) (layer "F.Cu") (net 6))
 (segment (start 151.685 116.535) (end 151.685 115.3821) (width 0.2) (layer "F.Cu") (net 6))
 (segment (start 157.690691 100.329) (end 158.909309 100.329) (width 0.2) (layer "F.Cu") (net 6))
 (segment (start 156.829 101.190691) (end 157.690691 100.329) (width 0.2) (layer "F.Cu") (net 6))
 (segment (start 151.685 115.3821) (end 156.829 110.2381) (width 0.2) (layer "F.Cu") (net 6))
 (segment (start 145.475 77.03) (end 146.25 77.03) (width 0.2) (layer "F.Cu") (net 6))
 (segment (start 118.269 104.236) (end 145.475 77.03) (width 0.2) (layer "F.Cu") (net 6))
 (segment (start 150.773068 120.901) (end 132.0839 120.901) (width 0.2) (layer "F.Cu") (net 6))
 (segment (start 159.771 101.190691) (end 159.771 111.903068) (width 0.2) (layer "F.Cu") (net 6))
 (segment (start 158.909309 100.329) (end 159.771 101.190691) (width 0.2) (layer "F.Cu") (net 6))
 (segment (start 118.269 107.0861) (end 118.269 104.236) (width 0.2) (layer "F.Cu") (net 6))
 (segment (start 159.771 111.903068) (end 150.773068 120.901) (width 0.2) (layer "F.Cu") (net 6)))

